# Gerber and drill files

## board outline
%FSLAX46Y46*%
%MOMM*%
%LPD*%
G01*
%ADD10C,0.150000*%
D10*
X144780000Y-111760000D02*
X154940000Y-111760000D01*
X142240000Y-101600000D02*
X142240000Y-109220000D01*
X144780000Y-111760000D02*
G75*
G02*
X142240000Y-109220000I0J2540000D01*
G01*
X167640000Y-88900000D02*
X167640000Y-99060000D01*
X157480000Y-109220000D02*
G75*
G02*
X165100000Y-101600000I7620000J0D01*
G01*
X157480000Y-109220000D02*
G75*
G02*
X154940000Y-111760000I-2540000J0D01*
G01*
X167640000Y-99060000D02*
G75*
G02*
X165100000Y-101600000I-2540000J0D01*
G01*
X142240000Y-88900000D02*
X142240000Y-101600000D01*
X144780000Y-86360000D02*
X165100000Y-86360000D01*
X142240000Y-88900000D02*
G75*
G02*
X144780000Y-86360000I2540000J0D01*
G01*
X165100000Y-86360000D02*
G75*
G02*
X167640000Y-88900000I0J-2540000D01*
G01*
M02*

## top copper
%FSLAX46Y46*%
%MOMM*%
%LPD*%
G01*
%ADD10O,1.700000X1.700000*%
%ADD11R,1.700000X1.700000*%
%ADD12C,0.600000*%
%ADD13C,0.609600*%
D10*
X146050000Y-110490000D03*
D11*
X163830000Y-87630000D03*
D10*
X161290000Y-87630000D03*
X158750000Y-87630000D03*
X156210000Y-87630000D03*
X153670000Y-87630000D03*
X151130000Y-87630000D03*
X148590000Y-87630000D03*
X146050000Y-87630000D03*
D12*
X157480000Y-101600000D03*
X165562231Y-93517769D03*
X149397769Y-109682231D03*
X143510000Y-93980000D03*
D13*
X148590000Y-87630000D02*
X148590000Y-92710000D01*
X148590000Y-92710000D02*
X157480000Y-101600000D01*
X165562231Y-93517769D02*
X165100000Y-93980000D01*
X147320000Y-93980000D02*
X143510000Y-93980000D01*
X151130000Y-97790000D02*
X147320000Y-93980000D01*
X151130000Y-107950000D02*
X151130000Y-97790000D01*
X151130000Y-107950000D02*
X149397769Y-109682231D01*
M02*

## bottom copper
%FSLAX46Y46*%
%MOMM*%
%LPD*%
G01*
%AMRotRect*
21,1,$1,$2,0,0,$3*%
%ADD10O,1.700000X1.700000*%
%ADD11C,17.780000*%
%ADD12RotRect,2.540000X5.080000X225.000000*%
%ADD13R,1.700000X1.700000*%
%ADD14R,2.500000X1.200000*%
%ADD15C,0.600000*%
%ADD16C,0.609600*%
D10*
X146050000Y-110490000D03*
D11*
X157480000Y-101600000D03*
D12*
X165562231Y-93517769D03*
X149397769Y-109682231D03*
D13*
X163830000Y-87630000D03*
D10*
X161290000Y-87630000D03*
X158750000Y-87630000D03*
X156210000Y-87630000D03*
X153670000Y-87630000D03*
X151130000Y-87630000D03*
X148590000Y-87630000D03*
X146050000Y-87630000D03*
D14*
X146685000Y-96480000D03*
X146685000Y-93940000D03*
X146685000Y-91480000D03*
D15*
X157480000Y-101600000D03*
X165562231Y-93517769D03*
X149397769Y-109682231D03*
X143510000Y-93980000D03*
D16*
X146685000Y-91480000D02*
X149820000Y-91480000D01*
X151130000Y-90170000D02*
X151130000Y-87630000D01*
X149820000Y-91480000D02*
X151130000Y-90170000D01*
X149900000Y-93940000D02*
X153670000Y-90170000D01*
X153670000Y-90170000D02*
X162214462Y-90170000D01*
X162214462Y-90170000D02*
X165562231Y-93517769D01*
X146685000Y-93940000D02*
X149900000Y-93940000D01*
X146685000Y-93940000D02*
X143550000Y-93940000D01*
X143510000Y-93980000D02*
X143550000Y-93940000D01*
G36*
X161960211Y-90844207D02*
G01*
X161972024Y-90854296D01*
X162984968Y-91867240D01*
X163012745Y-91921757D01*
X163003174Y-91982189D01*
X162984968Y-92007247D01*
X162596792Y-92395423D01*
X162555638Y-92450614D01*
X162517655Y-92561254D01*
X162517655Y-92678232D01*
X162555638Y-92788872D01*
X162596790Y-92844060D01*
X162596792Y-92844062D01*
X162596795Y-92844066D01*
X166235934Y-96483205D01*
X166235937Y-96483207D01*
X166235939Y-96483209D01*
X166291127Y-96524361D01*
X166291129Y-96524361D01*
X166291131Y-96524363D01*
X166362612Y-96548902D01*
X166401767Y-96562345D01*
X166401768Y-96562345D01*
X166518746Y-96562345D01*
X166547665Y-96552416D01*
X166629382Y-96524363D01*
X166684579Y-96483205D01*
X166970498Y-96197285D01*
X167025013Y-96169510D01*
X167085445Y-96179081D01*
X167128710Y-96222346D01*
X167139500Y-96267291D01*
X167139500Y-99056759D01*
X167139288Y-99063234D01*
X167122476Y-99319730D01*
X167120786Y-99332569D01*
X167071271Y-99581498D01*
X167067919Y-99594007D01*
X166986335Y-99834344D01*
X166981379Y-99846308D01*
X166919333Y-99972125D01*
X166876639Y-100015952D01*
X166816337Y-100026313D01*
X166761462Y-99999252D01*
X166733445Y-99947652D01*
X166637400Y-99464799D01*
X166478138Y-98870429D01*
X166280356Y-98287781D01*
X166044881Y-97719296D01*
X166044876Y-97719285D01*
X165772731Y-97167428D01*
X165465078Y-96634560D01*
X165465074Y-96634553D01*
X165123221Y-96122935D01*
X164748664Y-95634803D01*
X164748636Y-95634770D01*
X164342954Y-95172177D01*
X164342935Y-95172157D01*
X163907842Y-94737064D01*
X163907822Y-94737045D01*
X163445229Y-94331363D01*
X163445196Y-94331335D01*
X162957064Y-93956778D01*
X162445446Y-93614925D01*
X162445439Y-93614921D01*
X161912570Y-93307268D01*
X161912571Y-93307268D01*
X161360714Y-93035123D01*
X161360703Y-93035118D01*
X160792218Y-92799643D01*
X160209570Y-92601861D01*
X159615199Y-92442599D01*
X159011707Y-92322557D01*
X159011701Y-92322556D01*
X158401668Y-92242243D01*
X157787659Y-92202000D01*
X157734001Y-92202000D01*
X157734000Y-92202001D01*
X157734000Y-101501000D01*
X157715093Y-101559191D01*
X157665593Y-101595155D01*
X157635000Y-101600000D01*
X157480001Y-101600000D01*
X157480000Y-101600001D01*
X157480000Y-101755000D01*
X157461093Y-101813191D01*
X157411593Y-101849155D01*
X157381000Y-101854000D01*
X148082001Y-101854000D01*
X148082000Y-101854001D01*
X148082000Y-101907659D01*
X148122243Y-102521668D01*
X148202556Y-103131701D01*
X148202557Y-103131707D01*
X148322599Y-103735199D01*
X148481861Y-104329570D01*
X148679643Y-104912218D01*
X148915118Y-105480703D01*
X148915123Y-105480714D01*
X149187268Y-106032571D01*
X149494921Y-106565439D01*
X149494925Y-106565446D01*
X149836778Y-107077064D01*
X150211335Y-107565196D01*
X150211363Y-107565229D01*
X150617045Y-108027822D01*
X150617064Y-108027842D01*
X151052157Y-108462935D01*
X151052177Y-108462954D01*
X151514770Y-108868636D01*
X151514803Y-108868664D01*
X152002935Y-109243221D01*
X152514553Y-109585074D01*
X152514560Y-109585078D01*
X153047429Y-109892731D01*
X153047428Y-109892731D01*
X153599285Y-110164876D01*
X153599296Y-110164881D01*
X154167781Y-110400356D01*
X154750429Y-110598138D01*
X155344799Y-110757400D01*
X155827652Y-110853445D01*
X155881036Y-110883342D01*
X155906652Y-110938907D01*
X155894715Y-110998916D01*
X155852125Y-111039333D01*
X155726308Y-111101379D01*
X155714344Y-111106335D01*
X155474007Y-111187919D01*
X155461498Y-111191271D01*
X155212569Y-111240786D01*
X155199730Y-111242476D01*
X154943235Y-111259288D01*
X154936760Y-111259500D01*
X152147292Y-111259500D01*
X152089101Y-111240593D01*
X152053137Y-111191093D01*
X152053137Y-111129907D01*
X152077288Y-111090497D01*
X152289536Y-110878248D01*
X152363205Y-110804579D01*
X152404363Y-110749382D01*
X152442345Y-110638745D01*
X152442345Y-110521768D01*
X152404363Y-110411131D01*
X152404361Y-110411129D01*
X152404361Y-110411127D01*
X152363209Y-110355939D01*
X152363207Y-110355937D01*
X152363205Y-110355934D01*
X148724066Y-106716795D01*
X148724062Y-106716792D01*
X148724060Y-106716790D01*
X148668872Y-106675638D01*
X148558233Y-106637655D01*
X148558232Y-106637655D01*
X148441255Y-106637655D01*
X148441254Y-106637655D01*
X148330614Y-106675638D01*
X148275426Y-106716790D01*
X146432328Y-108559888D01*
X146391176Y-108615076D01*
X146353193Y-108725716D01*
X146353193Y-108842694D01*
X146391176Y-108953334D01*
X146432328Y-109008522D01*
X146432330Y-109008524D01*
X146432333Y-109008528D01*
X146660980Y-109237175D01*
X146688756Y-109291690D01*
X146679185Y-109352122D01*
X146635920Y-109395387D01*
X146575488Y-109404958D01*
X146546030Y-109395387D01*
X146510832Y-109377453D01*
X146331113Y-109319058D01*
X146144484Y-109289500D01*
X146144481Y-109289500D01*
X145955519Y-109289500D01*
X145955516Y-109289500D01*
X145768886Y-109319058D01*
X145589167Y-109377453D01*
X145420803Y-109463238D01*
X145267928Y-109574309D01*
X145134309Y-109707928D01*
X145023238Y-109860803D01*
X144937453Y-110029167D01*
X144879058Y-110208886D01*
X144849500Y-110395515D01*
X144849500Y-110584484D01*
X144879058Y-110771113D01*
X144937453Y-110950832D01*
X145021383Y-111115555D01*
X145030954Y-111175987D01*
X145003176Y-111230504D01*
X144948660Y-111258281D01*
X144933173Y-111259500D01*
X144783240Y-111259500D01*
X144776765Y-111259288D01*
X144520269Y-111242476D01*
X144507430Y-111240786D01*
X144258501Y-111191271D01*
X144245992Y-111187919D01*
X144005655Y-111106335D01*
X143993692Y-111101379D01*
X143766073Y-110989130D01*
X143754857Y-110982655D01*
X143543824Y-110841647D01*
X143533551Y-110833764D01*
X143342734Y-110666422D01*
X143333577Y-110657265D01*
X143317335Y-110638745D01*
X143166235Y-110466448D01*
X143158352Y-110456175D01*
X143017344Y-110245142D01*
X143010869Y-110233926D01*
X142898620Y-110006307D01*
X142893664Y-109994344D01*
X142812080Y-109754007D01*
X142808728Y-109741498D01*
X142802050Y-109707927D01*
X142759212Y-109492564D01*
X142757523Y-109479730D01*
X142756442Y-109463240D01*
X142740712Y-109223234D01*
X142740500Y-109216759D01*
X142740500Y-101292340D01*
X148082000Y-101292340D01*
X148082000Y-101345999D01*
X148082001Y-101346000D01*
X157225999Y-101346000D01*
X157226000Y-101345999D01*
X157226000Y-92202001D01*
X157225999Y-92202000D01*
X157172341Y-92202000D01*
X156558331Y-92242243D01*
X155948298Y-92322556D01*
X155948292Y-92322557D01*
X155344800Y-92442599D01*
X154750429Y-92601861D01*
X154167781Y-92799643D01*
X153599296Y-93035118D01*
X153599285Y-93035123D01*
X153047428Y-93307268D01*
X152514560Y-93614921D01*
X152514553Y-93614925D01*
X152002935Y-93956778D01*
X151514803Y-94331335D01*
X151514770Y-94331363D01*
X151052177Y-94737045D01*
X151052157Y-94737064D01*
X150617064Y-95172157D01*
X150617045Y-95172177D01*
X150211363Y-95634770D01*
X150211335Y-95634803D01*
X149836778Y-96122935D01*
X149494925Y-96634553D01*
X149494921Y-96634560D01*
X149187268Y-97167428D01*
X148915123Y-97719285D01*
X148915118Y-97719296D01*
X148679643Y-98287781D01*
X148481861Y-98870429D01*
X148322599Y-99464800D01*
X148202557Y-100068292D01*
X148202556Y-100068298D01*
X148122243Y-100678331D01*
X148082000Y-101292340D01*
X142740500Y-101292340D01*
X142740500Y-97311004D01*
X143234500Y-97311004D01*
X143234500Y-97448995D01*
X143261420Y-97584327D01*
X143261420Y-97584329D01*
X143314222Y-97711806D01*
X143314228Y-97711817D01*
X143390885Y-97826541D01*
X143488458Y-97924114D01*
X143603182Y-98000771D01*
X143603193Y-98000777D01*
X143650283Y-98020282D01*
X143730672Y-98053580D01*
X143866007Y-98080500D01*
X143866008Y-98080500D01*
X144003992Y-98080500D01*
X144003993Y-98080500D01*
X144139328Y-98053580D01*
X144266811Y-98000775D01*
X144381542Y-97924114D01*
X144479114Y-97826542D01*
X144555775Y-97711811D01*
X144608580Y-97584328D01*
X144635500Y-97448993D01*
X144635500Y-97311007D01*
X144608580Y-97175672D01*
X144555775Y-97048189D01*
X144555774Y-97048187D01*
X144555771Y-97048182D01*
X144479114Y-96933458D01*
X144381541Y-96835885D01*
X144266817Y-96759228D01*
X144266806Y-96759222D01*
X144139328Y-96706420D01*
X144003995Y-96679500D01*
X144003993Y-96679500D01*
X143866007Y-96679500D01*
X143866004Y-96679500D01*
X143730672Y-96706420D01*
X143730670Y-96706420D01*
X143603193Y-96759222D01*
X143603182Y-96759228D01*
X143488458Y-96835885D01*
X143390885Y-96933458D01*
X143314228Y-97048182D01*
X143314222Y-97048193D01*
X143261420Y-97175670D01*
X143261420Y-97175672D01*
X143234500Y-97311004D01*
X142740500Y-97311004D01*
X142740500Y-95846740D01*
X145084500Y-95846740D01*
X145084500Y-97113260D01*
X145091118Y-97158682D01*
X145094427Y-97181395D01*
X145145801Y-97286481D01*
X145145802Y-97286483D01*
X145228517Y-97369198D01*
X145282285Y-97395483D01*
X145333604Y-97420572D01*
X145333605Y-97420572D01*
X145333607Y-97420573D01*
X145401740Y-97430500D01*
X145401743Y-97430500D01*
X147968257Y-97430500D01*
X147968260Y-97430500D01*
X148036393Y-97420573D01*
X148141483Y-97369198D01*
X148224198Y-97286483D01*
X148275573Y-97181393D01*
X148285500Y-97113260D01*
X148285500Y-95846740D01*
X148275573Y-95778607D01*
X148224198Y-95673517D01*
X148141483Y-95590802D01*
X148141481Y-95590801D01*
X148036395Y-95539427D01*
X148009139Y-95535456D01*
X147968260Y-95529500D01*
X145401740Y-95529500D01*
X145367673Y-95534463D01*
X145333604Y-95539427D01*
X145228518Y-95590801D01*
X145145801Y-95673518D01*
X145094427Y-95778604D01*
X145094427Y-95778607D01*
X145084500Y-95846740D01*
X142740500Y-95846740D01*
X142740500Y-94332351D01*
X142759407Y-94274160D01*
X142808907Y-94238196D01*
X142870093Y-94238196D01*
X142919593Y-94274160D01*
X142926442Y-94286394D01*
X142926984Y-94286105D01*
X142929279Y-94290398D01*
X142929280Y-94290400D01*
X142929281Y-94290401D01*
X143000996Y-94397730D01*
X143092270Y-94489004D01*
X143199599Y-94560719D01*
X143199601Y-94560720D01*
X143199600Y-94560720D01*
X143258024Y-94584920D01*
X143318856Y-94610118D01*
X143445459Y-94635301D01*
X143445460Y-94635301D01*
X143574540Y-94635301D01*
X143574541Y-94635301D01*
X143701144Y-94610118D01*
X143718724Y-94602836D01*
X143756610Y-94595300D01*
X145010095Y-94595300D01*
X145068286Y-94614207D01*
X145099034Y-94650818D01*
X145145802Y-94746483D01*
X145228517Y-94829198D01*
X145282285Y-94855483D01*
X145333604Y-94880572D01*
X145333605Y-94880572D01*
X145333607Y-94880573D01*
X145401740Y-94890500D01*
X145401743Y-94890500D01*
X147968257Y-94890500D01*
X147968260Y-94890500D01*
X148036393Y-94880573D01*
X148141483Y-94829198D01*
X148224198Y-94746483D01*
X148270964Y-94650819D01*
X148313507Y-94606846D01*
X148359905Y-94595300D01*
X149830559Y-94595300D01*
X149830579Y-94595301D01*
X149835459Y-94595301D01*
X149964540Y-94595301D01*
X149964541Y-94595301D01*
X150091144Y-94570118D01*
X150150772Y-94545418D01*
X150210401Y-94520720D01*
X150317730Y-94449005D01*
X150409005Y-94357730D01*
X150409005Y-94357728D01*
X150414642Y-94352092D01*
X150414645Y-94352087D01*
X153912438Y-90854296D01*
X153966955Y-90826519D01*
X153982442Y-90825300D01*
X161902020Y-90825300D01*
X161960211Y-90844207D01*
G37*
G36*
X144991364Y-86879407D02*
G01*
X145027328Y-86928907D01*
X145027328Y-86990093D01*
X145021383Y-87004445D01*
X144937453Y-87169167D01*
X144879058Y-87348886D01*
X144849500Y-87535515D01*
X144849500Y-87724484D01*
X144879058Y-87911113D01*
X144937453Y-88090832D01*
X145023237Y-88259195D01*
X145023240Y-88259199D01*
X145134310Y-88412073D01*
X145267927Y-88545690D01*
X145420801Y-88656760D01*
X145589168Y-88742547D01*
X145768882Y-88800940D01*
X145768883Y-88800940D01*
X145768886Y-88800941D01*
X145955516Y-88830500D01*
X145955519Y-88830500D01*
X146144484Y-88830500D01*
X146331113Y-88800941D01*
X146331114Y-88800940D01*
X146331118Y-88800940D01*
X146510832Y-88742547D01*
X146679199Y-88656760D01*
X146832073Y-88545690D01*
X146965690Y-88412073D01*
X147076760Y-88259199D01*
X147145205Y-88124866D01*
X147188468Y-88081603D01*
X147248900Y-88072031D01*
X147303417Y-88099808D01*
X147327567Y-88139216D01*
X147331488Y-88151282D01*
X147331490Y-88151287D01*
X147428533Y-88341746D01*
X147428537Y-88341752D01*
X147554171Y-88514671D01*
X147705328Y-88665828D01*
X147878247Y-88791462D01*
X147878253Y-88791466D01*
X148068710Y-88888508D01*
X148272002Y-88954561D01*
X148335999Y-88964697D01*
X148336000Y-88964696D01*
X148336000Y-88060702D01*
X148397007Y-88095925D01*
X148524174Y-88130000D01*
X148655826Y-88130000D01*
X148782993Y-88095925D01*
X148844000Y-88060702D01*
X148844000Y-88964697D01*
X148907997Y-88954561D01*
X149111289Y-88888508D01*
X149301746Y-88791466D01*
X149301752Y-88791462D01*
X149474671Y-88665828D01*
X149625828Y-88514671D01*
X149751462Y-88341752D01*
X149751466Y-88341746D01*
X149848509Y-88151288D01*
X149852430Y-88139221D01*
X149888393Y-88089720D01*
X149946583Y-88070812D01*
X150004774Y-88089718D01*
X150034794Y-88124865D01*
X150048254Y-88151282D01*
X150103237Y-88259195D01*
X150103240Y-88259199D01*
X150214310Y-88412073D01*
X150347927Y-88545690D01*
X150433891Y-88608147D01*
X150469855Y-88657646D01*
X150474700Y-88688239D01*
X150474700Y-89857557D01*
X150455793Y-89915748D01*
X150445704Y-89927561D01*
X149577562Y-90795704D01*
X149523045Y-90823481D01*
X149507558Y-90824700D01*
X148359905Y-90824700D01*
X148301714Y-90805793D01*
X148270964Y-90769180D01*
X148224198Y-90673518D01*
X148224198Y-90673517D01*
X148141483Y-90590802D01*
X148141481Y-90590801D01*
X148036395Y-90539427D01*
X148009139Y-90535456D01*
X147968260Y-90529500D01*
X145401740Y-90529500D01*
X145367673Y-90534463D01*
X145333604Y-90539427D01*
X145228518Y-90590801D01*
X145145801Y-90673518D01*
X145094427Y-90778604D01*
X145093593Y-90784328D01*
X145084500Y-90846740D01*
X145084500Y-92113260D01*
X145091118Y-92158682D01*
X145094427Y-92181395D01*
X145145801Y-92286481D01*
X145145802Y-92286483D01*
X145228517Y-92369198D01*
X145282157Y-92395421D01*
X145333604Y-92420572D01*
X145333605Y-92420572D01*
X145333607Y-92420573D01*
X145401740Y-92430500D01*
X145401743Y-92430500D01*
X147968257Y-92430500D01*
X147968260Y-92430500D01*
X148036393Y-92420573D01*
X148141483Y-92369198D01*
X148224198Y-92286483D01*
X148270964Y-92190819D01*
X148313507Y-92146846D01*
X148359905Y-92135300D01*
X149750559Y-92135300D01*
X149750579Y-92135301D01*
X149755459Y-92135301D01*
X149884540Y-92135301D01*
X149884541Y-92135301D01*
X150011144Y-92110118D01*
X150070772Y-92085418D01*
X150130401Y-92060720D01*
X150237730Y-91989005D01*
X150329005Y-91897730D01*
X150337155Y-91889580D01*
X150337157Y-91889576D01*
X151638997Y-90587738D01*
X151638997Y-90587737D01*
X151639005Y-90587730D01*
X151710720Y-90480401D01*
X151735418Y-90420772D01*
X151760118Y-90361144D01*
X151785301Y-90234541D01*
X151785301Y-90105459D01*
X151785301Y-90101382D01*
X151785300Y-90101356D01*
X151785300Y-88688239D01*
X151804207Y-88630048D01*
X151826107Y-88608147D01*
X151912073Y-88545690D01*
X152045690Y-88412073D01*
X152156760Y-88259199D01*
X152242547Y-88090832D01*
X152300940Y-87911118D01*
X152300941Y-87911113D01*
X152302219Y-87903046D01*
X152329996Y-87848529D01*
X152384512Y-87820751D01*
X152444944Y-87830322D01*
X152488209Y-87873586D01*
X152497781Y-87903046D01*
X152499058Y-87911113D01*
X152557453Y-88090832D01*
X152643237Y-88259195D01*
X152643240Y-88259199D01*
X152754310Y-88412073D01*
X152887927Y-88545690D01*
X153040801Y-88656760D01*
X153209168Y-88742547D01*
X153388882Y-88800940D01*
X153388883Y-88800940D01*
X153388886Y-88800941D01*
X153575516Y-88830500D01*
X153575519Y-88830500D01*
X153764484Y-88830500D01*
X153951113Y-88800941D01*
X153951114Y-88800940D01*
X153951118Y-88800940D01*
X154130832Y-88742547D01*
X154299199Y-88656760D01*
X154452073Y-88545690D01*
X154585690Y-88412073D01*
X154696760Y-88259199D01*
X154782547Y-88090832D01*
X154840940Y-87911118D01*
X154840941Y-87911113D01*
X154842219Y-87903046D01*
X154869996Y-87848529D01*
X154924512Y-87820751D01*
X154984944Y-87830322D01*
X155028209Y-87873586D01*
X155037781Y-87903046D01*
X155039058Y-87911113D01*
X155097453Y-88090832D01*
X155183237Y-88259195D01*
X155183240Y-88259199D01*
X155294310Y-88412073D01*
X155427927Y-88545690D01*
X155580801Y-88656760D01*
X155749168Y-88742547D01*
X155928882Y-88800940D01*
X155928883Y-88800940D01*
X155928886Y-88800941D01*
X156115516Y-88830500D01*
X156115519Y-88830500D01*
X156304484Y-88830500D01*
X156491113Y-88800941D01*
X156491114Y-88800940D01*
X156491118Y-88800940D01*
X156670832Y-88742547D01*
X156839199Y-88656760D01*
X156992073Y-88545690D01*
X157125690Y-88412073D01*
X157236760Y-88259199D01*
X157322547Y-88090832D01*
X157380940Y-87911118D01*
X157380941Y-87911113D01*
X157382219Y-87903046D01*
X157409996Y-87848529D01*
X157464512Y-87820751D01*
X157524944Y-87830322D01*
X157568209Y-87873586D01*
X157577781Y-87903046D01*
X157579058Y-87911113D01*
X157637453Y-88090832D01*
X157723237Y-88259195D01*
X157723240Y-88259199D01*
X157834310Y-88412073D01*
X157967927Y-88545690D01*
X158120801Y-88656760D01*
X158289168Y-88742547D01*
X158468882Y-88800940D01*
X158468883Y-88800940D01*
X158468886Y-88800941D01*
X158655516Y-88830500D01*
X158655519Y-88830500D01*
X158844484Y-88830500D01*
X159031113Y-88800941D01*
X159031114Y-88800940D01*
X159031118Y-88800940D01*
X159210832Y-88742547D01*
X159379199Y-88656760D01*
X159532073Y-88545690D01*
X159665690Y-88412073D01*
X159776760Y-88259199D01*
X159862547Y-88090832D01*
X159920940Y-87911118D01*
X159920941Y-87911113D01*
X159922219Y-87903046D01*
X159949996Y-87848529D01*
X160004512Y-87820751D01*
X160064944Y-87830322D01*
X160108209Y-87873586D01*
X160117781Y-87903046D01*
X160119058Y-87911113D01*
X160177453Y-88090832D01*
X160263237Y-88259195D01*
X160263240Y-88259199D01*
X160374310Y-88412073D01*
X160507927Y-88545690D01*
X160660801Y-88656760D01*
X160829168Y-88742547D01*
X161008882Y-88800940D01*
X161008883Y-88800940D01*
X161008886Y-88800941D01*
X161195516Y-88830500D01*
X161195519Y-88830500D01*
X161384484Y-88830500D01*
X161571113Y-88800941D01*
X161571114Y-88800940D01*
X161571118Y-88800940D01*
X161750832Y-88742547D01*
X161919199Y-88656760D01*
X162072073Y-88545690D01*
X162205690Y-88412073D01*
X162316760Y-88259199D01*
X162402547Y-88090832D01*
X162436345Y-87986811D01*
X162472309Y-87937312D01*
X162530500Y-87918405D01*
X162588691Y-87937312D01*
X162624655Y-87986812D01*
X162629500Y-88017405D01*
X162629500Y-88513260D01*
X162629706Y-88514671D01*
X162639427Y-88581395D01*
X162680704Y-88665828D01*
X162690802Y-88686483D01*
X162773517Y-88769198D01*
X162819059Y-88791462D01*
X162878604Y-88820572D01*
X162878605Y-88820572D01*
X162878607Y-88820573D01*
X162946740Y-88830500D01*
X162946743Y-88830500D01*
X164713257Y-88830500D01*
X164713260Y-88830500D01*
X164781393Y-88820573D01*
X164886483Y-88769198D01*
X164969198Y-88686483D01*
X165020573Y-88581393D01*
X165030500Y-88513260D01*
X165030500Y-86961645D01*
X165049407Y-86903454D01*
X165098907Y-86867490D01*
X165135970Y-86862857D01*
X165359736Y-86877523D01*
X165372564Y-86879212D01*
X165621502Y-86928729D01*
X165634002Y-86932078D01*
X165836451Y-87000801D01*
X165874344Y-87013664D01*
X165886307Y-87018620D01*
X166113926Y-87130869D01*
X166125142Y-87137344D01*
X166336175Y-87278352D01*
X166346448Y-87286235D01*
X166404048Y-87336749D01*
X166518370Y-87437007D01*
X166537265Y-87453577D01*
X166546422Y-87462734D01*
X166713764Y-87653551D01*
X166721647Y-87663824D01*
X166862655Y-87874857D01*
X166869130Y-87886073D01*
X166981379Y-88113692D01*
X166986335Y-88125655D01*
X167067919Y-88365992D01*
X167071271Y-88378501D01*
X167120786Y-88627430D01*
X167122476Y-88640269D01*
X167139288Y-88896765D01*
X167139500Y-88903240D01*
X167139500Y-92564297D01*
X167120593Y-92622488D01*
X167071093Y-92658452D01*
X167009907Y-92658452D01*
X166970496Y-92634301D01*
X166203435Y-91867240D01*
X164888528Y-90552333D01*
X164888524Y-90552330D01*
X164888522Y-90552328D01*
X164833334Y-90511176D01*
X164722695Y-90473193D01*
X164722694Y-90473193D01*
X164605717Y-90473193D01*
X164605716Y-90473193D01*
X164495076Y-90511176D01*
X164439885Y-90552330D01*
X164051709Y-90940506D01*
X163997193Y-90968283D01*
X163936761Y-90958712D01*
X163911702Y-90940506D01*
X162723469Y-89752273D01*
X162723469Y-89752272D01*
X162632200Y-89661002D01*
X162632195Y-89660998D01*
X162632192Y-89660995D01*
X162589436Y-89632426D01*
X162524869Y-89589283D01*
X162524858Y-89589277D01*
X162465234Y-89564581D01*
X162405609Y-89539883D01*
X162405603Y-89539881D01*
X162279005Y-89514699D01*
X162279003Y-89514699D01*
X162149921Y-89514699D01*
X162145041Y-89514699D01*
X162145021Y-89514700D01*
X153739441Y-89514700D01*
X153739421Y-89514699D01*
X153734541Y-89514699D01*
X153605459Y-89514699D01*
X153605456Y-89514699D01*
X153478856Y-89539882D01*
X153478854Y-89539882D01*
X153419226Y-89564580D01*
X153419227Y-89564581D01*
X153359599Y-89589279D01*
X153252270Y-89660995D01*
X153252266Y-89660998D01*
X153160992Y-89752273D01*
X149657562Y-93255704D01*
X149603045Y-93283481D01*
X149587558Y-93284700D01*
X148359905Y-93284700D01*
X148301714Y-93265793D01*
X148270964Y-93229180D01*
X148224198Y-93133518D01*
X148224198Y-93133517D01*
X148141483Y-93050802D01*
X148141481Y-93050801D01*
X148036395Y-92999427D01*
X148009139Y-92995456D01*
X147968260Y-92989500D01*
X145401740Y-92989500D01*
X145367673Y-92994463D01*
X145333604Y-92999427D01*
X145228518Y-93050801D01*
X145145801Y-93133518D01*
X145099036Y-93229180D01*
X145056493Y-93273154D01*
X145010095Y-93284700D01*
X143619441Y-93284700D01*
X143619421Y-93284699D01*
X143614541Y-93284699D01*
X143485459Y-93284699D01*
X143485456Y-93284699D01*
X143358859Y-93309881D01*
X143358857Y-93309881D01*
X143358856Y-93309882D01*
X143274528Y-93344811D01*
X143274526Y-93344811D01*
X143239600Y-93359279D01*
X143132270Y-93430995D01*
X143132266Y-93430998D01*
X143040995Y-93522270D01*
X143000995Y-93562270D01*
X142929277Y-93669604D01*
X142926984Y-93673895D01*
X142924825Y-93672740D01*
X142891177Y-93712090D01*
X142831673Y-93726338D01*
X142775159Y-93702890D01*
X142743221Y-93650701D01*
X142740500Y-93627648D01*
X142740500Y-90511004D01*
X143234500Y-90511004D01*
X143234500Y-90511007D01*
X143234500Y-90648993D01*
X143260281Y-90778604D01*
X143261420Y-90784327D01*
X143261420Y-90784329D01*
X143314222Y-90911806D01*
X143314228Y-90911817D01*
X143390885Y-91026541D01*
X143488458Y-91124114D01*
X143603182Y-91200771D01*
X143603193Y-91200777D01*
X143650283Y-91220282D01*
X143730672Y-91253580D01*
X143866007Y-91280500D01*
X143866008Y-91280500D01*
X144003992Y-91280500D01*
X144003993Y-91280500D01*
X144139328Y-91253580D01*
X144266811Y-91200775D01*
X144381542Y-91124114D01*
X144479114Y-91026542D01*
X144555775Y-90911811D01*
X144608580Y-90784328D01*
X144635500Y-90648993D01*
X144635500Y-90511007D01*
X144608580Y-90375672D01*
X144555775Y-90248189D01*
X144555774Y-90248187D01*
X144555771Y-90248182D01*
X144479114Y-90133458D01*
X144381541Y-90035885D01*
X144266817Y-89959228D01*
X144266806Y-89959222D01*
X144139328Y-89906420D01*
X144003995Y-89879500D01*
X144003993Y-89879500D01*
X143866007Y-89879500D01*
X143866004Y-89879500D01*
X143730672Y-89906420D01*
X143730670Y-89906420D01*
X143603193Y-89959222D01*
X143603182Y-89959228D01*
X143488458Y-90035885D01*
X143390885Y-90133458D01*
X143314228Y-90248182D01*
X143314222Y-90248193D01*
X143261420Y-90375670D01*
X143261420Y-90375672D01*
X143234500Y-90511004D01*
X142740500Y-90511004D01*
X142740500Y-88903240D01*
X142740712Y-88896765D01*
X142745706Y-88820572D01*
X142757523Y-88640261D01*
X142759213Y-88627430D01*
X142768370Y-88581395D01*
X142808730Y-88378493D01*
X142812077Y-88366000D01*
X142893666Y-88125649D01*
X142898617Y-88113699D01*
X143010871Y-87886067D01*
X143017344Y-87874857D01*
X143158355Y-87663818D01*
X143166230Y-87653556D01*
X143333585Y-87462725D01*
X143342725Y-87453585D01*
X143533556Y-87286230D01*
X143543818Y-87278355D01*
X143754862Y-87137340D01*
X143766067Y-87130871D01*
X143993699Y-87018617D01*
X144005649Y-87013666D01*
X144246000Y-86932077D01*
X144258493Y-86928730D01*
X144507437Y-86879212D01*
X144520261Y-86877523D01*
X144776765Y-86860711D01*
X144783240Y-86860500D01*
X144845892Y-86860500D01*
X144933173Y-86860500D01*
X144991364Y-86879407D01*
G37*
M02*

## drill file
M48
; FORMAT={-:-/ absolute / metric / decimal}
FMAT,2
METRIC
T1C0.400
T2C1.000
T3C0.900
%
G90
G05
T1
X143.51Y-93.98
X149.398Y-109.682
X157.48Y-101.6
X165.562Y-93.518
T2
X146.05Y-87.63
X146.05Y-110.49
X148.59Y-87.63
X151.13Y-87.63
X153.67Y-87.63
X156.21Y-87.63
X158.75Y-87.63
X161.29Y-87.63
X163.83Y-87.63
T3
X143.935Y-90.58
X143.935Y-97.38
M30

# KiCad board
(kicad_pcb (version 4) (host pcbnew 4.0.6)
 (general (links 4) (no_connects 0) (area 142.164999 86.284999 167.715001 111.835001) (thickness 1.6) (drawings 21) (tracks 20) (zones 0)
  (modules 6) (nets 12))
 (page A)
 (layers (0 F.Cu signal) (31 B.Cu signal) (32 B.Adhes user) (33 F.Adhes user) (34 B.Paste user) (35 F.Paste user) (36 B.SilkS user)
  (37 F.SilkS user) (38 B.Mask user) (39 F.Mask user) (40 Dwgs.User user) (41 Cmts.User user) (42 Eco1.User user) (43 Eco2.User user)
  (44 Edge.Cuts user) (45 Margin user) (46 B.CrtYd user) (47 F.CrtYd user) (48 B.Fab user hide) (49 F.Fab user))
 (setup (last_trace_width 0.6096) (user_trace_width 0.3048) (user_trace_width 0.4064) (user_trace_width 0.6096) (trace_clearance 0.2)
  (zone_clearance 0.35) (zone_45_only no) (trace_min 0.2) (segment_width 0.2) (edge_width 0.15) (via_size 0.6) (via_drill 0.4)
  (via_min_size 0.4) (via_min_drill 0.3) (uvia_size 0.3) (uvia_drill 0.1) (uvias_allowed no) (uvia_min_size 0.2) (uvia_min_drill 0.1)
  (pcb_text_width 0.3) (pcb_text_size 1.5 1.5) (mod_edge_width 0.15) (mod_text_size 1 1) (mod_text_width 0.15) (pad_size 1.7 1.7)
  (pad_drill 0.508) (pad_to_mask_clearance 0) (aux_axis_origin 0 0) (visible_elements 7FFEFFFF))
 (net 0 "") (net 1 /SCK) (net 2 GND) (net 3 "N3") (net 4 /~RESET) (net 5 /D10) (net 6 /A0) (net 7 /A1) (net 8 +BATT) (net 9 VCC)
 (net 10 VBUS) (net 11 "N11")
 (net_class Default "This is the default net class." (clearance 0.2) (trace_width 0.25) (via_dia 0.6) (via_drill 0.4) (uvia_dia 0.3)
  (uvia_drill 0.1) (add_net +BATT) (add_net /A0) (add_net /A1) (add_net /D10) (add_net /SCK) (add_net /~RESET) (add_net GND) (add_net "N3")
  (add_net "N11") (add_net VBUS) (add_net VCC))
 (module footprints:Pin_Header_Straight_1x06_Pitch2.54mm (layer F.Cu) (at 158.75 110.49 270)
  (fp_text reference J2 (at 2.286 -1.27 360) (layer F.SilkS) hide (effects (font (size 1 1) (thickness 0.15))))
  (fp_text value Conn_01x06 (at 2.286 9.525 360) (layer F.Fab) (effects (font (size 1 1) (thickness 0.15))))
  (pad 6 thru_hole oval (at 0 12.7 270) (size 1.7 1.7) (drill 1) (layers *.Cu *.Mask) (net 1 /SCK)))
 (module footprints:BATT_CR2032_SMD (layer B.Cu) (at 157.48 101.6 225)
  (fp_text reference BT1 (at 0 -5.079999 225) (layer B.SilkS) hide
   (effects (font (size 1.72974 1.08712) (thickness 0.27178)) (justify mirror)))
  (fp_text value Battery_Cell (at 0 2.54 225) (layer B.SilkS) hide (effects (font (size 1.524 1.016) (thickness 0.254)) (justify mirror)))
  (pad 2 smd circle (at 0 0 225) (size 17.78 17.78) (layers B.Cu B.Paste B.Mask) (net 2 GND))
  (pad 1 smd rect (at -11.43 0 225) (size 2.54 5.08) (layers B.Cu B.Paste B.Mask) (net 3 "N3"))
  (pad 1 smd rect (at 11.43 0 225) (size 2.54 5.08) (layers B.Cu B.Paste B.Mask) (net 3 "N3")))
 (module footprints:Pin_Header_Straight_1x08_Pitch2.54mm (layer F.Cu) (at 163.83 87.63 270)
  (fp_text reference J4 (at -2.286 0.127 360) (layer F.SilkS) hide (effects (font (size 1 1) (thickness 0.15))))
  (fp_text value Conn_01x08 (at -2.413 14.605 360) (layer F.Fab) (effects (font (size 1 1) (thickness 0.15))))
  (pad 1 thru_hole rect (at 0 0 270) (size 1.7 1.7) (drill 1) (layers *.Cu *.Mask) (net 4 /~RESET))
  (pad 2 thru_hole oval (at 0 2.54 270) (size 1.7 1.7) (drill 1) (layers *.Cu *.Mask) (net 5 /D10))
  (pad 3 thru_hole oval (at 0 5.08 270) (size 1.7 1.7) (drill 1) (layers *.Cu *.Mask) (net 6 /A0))
  (pad 4 thru_hole oval (at 0 7.62 270) (size 1.7 1.7) (drill 1) (layers *.Cu *.Mask) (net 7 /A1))
  (pad 5 thru_hole oval (at 0 10.16 270) (size 1.7 1.7) (drill 1) (layers *.Cu *.Mask) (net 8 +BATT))
  (pad 6 thru_hole oval (at 0 12.7 270) (size 1.7 1.7) (drill 1) (layers *.Cu *.Mask) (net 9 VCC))
  (pad 7 thru_hole oval (at 0 15.24 270) (size 1.7 1.7) (drill 1) (layers *.Cu *.Mask) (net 2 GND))
  (pad 8 thru_hole oval (at 0 17.78 270) (size 1.7 1.7) (drill 1) (layers *.Cu *.Mask) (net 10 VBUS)))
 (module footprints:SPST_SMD (layer B.Cu) (at 146.685 93.98 90)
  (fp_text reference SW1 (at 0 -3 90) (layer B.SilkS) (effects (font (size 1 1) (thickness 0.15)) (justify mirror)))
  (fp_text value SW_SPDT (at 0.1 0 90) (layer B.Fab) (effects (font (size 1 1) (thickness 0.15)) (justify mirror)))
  (pad "" np_thru_hole circle (at 3.4 -2.75 90) (size 0.9 0.9) (drill 0.9) (layers *.Cu *.Mask))
  (pad 1 smd rect (at -2.5 0 90) (size 1.2 2.5) (layers B.Cu B.Paste B.Mask) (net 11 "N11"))
  (pad 2 smd rect (at 0.04 0 90) (size 1.2 2.5) (layers B.Cu B.Paste B.Mask) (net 3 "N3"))
  (pad 3 smd rect (at 2.5 0 90) (size 1.2 2.5) (layers B.Cu B.Paste B.Mask) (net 9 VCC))
  (pad "" np_thru_hole circle (at -3.4 -2.75 90) (size 0.9 0.9) (drill 0.9) (layers *.Cu *.Mask)))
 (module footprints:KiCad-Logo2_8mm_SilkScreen (layer F.Cu) (at 155.194 98.425)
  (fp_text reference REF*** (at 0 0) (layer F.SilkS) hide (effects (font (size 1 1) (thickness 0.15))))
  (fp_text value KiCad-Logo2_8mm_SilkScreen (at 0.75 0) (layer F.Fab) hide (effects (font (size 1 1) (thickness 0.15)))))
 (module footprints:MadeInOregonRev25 (layer B.Cu) (at 148.209 104.902 180)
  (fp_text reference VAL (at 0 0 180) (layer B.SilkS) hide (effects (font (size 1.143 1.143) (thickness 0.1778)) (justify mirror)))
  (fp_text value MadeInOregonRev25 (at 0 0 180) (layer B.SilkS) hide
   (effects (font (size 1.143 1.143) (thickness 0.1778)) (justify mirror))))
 (gr_line (start 144.78 111.76) (end 154.94 111.76) (angle 90) (layer Edge.Cuts) (width 0.15))
 (gr_line (start 142.24 101.6) (end 142.24 109.22) (angle 90) (layer Edge.Cuts) (width 0.15))
 (gr_arc (start 144.78 109.22) (end 144.78 111.76) (angle 90) (layer Edge.Cuts) (width 0.15))
 (gr_line (start 167.64 88.9) (end 167.64 99.06) (angle 90) (layer Edge.Cuts) (width 0.15))
 (gr_arc (start 165.1 109.22) (end 157.48 109.22) (angle 90) (layer Edge.Cuts) (width 0.15))
 (gr_arc (start 154.94 109.22) (end 157.48 109.22) (angle 90) (layer Edge.Cuts) (width 0.15))
 (gr_arc (start 165.1 99.06) (end 167.64 99.06) (angle 90) (layer Edge.Cuts) (width 0.15))
 (gr_line (start 142.24 88.9) (end 142.24 101.6) (angle 90) (layer Edge.Cuts) (width 0.15))
 (gr_line (start 144.78 86.36) (end 165.1 86.36) (angle 90) (layer Edge.Cuts) (width 0.15))
 (gr_arc (start 144.78 88.9) (end 142.24 88.9) (angle 90) (layer Edge.Cuts) (width 0.15))
 (gr_arc (start 165.1 88.9) (end 165.1 86.36) (angle 90) (layer Edge.Cuts) (width 0.15))
 (segment (start 148.59 87.63) (end 148.59 92.71) (width 0.6096) (layer F.Cu) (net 2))
 (via (at 157.48 101.6) (size 0.6) (drill 0.4) (layers F.Cu B.Cu) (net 2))
 (segment (start 148.59 92.71) (end 157.48 101.6) (width 0.6096) (layer F.Cu) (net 2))
 (segment (start 146.685 91.48) (end 149.82 91.48) (width 0.6096) (layer B.Cu) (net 9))
 (segment (start 151.13 90.17) (end 151.13 87.63) (width 0.6096) (layer B.Cu) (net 9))
 (segment (start 149.82 91.48) (end 151.13 90.17) (width 0.6096) (layer B.Cu) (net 9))
 (via (at 165.562231 93.517769) (size 0.6) (drill 0.4) (layers F.Cu B.Cu) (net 3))
 (segment (start 149.9 93.94) (end 153.67 90.17) (width 0.6096) (layer B.Cu) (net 3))
 (segment (start 153.67 90.17) (end 162.214462 90.17) (width 0.6096) (layer B.Cu) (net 3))
 (segment (start 162.214462 90.17) (end 165.562231 93.517769) (width 0.6096) (layer B.Cu) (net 3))
 (segment (start 146.685 93.94) (end 149.9 93.94) (width 0.6096) (layer B.Cu) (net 3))
 (segment (start 165.562231 93.517769) (end 165.1 93.98) (width 0.6096) (layer F.Cu) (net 3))
 (via (at 149.397769 109.682231) (size 0.6) (drill 0.4) (layers F.Cu B.Cu) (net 3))
 (segment (start 146.685 93.94) (end 143.55 93.94) (width 0.6096) (layer B.Cu) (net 3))
 (segment (start 143.51 93.98) (end 143.55 93.94) (width 0.6096) (layer B.Cu) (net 3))
 (via (at 143.51 93.98) (size 0.6) (drill 0.4) (layers F.Cu B.Cu) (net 3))
 (segment (start 147.32 93.98) (end 143.51 93.98) (width 0.6096) (layer F.Cu) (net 3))
 (segment (start 151.13 97.79) (end 147.32 93.98) (width 0.6096) (layer F.Cu) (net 3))
 (segment (start 151.13 107.95) (end 151.13 97.79) (width 0.6096) (layer F.Cu) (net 3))
 (segment (start 151.13 107.95) (end 149.397769 109.682231) (width 0.6096) (layer F.Cu) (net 3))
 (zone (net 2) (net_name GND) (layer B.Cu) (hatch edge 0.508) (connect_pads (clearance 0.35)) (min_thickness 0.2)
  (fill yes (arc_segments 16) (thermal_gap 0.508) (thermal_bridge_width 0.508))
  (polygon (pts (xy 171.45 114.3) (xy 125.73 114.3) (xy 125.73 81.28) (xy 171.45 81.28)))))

